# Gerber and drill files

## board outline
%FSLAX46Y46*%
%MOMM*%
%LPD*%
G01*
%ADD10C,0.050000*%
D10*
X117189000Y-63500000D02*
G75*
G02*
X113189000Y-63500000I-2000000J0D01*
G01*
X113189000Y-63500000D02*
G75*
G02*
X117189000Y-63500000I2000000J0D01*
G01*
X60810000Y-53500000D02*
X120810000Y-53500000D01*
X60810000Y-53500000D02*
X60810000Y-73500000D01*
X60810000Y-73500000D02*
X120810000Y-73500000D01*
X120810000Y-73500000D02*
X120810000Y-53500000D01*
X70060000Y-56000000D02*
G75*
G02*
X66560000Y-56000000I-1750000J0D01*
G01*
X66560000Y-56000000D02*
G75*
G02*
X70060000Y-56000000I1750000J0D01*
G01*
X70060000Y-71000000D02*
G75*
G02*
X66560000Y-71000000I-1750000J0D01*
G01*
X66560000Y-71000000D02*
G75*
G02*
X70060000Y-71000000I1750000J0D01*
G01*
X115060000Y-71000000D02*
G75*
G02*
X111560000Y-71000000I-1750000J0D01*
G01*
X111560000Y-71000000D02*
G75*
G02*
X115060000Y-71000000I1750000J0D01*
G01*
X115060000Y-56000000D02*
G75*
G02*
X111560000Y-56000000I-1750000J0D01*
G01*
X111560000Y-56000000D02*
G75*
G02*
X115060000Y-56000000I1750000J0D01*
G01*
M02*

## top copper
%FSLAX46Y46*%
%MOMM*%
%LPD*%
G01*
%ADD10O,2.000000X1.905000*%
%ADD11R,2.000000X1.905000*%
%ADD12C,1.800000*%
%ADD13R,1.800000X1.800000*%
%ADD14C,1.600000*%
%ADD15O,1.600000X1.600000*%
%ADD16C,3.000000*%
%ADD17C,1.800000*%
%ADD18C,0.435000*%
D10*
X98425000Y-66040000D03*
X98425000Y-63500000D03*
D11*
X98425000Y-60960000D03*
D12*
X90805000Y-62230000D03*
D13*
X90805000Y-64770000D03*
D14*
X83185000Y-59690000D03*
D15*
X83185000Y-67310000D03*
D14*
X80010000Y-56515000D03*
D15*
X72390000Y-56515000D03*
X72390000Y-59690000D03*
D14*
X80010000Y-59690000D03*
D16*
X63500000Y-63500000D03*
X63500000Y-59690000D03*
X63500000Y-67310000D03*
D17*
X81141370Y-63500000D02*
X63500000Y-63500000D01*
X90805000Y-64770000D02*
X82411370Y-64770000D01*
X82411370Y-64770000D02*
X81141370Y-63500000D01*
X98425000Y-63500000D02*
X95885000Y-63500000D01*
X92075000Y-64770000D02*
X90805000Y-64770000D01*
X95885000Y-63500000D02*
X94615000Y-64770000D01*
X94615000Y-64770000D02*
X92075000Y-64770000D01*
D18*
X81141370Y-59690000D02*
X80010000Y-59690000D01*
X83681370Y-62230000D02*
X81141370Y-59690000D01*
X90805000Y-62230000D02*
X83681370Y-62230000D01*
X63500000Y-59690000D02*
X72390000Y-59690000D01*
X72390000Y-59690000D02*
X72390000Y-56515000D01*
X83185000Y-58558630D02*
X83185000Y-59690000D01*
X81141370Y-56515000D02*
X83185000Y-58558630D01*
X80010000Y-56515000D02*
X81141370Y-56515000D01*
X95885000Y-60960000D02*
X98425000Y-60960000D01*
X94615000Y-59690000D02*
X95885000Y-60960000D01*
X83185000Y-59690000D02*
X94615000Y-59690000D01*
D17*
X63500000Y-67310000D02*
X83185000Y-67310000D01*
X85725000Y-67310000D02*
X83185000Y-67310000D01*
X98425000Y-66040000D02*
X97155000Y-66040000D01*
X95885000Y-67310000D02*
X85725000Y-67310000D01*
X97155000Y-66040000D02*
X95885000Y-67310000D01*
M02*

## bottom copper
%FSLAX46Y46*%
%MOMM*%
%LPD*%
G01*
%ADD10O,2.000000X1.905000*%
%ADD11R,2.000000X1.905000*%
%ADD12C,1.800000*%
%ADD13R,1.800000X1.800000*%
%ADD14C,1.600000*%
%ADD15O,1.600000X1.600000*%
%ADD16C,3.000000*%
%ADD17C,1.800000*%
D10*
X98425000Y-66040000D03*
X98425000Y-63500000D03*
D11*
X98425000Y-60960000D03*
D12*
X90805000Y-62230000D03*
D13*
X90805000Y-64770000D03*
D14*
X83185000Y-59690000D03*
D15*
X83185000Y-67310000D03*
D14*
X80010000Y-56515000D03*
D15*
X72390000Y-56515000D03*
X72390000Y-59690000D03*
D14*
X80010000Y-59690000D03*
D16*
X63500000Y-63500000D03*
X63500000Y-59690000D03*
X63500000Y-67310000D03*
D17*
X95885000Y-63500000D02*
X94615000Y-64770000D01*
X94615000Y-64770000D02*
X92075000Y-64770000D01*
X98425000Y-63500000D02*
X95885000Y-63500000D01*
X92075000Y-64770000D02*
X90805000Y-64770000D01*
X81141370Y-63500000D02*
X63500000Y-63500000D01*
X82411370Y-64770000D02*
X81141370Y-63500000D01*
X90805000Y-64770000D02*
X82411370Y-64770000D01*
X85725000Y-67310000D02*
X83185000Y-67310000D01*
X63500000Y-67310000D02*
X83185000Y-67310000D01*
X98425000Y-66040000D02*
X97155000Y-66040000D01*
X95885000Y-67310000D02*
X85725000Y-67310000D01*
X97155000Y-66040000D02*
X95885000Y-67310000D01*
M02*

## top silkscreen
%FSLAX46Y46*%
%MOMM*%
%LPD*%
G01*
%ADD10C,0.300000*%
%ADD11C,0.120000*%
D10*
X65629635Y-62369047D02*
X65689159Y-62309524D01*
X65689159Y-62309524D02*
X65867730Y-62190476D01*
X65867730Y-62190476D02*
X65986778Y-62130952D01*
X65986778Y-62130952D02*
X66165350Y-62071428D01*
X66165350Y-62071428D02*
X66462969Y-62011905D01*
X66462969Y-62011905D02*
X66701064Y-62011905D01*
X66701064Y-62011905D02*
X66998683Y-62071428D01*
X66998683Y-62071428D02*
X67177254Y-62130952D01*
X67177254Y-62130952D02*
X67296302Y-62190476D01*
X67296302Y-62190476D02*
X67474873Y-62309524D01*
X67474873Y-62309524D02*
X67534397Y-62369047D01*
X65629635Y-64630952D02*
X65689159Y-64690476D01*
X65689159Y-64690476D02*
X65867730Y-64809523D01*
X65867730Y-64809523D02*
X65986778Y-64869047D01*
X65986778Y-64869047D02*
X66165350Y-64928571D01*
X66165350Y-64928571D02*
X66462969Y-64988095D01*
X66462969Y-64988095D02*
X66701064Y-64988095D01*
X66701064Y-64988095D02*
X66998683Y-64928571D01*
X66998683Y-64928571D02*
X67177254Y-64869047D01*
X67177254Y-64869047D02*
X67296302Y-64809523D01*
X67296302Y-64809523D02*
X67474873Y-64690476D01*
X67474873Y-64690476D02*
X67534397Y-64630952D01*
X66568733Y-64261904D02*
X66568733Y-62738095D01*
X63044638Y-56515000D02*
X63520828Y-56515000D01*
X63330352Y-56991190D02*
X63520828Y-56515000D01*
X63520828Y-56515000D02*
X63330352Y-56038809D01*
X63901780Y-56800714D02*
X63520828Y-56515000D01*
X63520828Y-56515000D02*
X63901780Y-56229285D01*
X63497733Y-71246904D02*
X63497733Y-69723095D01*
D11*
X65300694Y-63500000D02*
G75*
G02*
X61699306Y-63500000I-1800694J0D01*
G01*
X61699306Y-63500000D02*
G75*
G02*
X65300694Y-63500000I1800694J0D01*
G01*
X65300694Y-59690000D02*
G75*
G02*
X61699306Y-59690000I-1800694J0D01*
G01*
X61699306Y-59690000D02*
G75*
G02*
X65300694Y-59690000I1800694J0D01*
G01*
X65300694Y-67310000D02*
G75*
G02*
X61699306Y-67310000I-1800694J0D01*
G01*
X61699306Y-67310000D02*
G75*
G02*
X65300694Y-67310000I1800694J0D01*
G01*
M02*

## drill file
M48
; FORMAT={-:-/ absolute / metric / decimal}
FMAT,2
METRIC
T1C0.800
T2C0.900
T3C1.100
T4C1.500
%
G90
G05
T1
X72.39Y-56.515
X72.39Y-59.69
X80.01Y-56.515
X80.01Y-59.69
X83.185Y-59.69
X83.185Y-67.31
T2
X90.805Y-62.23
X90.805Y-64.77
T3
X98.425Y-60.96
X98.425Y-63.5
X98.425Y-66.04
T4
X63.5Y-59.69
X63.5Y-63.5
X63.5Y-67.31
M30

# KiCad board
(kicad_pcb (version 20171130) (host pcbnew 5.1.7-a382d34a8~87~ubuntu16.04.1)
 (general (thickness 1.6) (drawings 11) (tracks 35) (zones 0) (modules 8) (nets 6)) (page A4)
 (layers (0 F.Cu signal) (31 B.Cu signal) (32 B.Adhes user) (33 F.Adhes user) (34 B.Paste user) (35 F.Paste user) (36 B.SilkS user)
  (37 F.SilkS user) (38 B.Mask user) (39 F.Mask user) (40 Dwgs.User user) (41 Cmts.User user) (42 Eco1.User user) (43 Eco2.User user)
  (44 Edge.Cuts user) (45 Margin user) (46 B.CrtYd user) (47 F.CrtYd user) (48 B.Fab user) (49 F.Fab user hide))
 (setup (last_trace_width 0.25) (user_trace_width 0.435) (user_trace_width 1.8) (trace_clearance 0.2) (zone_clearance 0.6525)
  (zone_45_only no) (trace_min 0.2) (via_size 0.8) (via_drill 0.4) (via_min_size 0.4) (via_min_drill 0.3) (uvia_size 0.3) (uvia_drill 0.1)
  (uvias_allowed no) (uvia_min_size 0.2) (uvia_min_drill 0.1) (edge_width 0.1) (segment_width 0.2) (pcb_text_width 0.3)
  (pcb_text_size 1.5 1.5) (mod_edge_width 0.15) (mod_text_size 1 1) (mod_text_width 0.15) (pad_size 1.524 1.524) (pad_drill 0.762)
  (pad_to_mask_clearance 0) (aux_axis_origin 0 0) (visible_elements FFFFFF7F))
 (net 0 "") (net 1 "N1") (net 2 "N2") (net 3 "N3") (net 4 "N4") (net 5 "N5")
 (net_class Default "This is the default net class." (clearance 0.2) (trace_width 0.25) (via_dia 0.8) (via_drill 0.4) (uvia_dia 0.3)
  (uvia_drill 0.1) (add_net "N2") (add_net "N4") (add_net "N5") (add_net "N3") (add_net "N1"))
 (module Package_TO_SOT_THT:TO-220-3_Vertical (layer F.Cu) (at 98.425 60.96 270)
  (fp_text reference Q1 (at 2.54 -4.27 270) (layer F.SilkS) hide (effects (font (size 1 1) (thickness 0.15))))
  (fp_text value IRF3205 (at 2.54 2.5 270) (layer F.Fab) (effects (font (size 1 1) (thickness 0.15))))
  (pad 3 thru_hole oval (at 5.08 0 270) (size 1.905 2) (drill 1.1) (layers *.Cu *.Mask) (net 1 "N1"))
  (pad 2 thru_hole oval (at 2.54 0 270) (size 1.905 2) (drill 1.1) (layers *.Cu *.Mask) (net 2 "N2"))
  (pad 1 thru_hole rect (at 0 0 270) (size 1.905 2) (drill 1.1) (layers *.Cu *.Mask) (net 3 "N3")))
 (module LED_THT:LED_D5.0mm (layer F.Cu) (at 90.805 64.77 90)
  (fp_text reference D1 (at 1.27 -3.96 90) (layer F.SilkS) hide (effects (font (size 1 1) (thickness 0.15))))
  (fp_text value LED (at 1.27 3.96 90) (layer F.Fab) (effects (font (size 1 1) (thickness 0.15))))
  (pad 2 thru_hole circle (at 2.54 0 90) (size 1.8 1.8) (drill 0.9) (layers *.Cu *.Mask) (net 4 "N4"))
  (pad 1 thru_hole rect (at 0 0 90) (size 1.8 1.8) (drill 0.9) (layers *.Cu *.Mask) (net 2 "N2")))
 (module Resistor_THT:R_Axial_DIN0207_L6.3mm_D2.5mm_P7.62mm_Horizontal (layer F.Cu) (at 83.185 59.69 270)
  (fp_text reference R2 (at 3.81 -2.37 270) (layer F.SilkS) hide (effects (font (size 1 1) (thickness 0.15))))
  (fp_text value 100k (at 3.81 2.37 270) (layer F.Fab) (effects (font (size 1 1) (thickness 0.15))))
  (pad 1 thru_hole circle (at 0 0 270) (size 1.6 1.6) (drill 0.8) (layers *.Cu *.Mask) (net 3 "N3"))
  (pad 2 thru_hole oval (at 7.62 0 270) (size 1.6 1.6) (drill 0.8) (layers *.Cu *.Mask) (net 1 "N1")))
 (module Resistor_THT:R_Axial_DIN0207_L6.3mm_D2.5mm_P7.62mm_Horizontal (layer F.Cu) (at 80.01 56.515 180)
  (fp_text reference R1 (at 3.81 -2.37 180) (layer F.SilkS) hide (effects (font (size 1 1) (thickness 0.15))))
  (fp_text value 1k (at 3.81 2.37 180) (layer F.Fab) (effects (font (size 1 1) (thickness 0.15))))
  (pad 1 thru_hole circle (at 0 0 180) (size 1.6 1.6) (drill 0.8) (layers *.Cu *.Mask) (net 3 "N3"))
  (pad 2 thru_hole oval (at 7.62 0 180) (size 1.6 1.6) (drill 0.8) (layers *.Cu *.Mask) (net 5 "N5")))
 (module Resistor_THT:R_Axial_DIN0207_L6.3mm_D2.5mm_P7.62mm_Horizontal (layer F.Cu) (at 80.01 59.69 180)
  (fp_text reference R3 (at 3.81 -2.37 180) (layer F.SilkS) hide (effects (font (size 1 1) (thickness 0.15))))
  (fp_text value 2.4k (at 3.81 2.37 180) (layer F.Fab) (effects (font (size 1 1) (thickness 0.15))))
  (pad 2 thru_hole oval (at 7.62 0 180) (size 1.6 1.6) (drill 0.8) (layers *.Cu *.Mask) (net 5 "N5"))
  (pad 1 thru_hole circle (at 0 0 180) (size 1.6 1.6) (drill 0.8) (layers *.Cu *.Mask) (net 4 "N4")))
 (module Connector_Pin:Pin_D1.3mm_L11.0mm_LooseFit (layer F.Cu) (at 63.5 63.5)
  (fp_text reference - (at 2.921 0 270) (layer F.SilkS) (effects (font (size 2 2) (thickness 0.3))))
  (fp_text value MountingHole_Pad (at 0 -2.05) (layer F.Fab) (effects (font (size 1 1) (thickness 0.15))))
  (fp_circle (center 0 0) (end 1.8 0.05) (layer F.SilkS) (width 0.12))
  (pad 1 thru_hole circle (at 0 0) (size 3 3) (drill 1.5) (layers *.Cu *.Mask) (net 2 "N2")))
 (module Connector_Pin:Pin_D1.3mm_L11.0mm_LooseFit (layer F.Cu) (at 63.5 59.69)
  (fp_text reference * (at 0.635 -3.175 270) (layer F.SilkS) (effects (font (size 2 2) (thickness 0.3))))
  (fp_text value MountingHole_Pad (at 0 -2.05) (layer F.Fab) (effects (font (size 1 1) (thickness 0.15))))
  (fp_circle (center 0 0) (end 1.8 0.05) (layer F.SilkS) (width 0.12))
  (pad 1 thru_hole circle (at 0 0) (size 3 3) (drill 1.5) (layers *.Cu *.Mask) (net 5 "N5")))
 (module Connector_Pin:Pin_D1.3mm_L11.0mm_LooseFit (layer F.Cu) (at 63.5 67.31)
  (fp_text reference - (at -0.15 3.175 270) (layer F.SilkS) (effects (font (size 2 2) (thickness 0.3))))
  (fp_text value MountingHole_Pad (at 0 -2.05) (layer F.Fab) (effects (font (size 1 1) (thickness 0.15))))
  (fp_circle (center 0 0) (end 1.8 0.05) (layer F.SilkS) (width 0.12))
  (pad 1 thru_hole circle (at 0 0) (size 3 3) (drill 1.5) (layers *.Cu *.Mask) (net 1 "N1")))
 (gr_circle (center 115.189 63.5) (end 117.189 63.5) (layer Edge.Cuts) (width 0.05))
 (gr_line (start 60.81 53.5) (end 120.81 53.5) (layer Edge.Cuts) (width 0.05))
 (gr_line (start 60.81 53.5) (end 60.81 73.5) (layer Edge.Cuts) (width 0.05))
 (gr_line (start 60.81 73.5) (end 120.81 73.5) (layer Edge.Cuts) (width 0.05))
 (gr_line (start 120.81 73.5) (end 120.81 53.5) (layer Edge.Cuts) (width 0.05))
 (gr_circle (center 68.31 56) (end 70.06 56) (layer Edge.Cuts) (width 0.05))
 (gr_circle (center 68.31 71) (end 70.06 71) (layer Edge.Cuts) (width 0.05))
 (gr_circle (center 113.31 71) (end 115.06 71) (layer Edge.Cuts) (width 0.05))
 (gr_circle (center 113.31 56) (end 115.06 56) (layer Edge.Cuts) (width 0.05))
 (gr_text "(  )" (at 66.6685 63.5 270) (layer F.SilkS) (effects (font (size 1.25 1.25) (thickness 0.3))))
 (segment (start 81.14137 63.5) (end 63.5 63.5) (width 1.8) (layer F.Cu) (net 2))
 (segment (start 90.805 64.77) (end 82.41137 64.77) (width 1.8) (layer F.Cu) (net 2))
 (segment (start 82.41137 64.77) (end 81.14137 63.5) (width 1.8) (layer F.Cu) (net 2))
 (segment (start 98.425 63.5) (end 95.885 63.5) (width 1.8) (layer F.Cu) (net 2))
 (segment (start 92.075 64.77) (end 90.805 64.77) (width 1.8) (layer F.Cu) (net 2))
 (segment (start 95.885 63.5) (end 94.615 64.77) (width 1.8) (layer F.Cu) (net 2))
 (segment (start 94.615 64.77) (end 92.075 64.77) (width 1.8) (layer F.Cu) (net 2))
 (segment (start 95.885 63.5) (end 94.615 64.77) (width 1.8) (layer B.Cu) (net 2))
 (segment (start 94.615 64.77) (end 92.075 64.77) (width 1.8) (layer B.Cu) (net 2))
 (segment (start 98.425 63.5) (end 95.885 63.5) (width 1.8) (layer B.Cu) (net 2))
 (segment (start 92.075 64.77) (end 90.805 64.77) (width 1.8) (layer B.Cu) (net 2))
 (segment (start 81.14137 63.5) (end 63.5 63.5) (width 1.8) (layer B.Cu) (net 2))
 (segment (start 82.41137 64.77) (end 81.14137 63.5) (width 1.8) (layer B.Cu) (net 2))
 (segment (start 90.805 64.77) (end 82.41137 64.77) (width 1.8) (layer B.Cu) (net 2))
 (segment (start 81.14137 59.69) (end 80.01 59.69) (width 0.435) (layer F.Cu) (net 4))
 (segment (start 83.68137 62.23) (end 81.14137 59.69) (width 0.435) (layer F.Cu) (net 4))
 (segment (start 90.805 62.23) (end 83.68137 62.23) (width 0.435) (layer F.Cu) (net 4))
 (segment (start 63.5 59.69) (end 72.39 59.69) (width 0.435) (layer F.Cu) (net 5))
 (segment (start 72.39 59.69) (end 72.39 56.515) (width 0.435) (layer F.Cu) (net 5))
 (segment (start 83.185 58.55863) (end 83.185 59.69) (width 0.435) (layer F.Cu) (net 3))
 (segment (start 81.14137 56.515) (end 83.185 58.55863) (width 0.435) (layer F.Cu) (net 3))
 (segment (start 80.01 56.515) (end 81.14137 56.515) (width 0.435) (layer F.Cu) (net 3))
 (segment (start 95.885 60.96) (end 98.425 60.96) (width 0.435) (layer F.Cu) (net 3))
 (segment (start 94.615 59.69) (end 95.885 60.96) (width 0.435) (layer F.Cu) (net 3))
 (segment (start 83.185 59.69) (end 94.615 59.69) (width 0.435) (layer F.Cu) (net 3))
 (segment (start 63.5 67.31) (end 83.185 67.31) (width 1.8) (layer F.Cu) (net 1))
 (segment (start 85.725 67.31) (end 83.185 67.31) (width 1.8) (layer F.Cu) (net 1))
 (segment (start 98.425 66.04) (end 97.155 66.04) (width 1.8) (layer F.Cu) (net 1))
 (segment (start 95.885 67.31) (end 85.725 67.31) (width 1.8) (layer F.Cu) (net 1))
 (segment (start 97.155 66.04) (end 95.885 67.31) (width 1.8) (layer F.Cu) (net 1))
 (segment (start 85.725 67.31) (end 83.185 67.31) (width 1.8) (layer B.Cu) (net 1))
 (segment (start 63.5 67.31) (end 83.185 67.31) (width 1.8) (layer B.Cu) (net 1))
 (segment (start 98.425 66.04) (end 97.155 66.04) (width 1.8) (layer B.Cu) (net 1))
 (segment (start 95.885 67.31) (end 85.725 67.31) (width 1.8) (layer B.Cu) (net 1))
 (segment (start 97.155 66.04) (end 95.885 67.31) (width 1.8) (layer B.Cu) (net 1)))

